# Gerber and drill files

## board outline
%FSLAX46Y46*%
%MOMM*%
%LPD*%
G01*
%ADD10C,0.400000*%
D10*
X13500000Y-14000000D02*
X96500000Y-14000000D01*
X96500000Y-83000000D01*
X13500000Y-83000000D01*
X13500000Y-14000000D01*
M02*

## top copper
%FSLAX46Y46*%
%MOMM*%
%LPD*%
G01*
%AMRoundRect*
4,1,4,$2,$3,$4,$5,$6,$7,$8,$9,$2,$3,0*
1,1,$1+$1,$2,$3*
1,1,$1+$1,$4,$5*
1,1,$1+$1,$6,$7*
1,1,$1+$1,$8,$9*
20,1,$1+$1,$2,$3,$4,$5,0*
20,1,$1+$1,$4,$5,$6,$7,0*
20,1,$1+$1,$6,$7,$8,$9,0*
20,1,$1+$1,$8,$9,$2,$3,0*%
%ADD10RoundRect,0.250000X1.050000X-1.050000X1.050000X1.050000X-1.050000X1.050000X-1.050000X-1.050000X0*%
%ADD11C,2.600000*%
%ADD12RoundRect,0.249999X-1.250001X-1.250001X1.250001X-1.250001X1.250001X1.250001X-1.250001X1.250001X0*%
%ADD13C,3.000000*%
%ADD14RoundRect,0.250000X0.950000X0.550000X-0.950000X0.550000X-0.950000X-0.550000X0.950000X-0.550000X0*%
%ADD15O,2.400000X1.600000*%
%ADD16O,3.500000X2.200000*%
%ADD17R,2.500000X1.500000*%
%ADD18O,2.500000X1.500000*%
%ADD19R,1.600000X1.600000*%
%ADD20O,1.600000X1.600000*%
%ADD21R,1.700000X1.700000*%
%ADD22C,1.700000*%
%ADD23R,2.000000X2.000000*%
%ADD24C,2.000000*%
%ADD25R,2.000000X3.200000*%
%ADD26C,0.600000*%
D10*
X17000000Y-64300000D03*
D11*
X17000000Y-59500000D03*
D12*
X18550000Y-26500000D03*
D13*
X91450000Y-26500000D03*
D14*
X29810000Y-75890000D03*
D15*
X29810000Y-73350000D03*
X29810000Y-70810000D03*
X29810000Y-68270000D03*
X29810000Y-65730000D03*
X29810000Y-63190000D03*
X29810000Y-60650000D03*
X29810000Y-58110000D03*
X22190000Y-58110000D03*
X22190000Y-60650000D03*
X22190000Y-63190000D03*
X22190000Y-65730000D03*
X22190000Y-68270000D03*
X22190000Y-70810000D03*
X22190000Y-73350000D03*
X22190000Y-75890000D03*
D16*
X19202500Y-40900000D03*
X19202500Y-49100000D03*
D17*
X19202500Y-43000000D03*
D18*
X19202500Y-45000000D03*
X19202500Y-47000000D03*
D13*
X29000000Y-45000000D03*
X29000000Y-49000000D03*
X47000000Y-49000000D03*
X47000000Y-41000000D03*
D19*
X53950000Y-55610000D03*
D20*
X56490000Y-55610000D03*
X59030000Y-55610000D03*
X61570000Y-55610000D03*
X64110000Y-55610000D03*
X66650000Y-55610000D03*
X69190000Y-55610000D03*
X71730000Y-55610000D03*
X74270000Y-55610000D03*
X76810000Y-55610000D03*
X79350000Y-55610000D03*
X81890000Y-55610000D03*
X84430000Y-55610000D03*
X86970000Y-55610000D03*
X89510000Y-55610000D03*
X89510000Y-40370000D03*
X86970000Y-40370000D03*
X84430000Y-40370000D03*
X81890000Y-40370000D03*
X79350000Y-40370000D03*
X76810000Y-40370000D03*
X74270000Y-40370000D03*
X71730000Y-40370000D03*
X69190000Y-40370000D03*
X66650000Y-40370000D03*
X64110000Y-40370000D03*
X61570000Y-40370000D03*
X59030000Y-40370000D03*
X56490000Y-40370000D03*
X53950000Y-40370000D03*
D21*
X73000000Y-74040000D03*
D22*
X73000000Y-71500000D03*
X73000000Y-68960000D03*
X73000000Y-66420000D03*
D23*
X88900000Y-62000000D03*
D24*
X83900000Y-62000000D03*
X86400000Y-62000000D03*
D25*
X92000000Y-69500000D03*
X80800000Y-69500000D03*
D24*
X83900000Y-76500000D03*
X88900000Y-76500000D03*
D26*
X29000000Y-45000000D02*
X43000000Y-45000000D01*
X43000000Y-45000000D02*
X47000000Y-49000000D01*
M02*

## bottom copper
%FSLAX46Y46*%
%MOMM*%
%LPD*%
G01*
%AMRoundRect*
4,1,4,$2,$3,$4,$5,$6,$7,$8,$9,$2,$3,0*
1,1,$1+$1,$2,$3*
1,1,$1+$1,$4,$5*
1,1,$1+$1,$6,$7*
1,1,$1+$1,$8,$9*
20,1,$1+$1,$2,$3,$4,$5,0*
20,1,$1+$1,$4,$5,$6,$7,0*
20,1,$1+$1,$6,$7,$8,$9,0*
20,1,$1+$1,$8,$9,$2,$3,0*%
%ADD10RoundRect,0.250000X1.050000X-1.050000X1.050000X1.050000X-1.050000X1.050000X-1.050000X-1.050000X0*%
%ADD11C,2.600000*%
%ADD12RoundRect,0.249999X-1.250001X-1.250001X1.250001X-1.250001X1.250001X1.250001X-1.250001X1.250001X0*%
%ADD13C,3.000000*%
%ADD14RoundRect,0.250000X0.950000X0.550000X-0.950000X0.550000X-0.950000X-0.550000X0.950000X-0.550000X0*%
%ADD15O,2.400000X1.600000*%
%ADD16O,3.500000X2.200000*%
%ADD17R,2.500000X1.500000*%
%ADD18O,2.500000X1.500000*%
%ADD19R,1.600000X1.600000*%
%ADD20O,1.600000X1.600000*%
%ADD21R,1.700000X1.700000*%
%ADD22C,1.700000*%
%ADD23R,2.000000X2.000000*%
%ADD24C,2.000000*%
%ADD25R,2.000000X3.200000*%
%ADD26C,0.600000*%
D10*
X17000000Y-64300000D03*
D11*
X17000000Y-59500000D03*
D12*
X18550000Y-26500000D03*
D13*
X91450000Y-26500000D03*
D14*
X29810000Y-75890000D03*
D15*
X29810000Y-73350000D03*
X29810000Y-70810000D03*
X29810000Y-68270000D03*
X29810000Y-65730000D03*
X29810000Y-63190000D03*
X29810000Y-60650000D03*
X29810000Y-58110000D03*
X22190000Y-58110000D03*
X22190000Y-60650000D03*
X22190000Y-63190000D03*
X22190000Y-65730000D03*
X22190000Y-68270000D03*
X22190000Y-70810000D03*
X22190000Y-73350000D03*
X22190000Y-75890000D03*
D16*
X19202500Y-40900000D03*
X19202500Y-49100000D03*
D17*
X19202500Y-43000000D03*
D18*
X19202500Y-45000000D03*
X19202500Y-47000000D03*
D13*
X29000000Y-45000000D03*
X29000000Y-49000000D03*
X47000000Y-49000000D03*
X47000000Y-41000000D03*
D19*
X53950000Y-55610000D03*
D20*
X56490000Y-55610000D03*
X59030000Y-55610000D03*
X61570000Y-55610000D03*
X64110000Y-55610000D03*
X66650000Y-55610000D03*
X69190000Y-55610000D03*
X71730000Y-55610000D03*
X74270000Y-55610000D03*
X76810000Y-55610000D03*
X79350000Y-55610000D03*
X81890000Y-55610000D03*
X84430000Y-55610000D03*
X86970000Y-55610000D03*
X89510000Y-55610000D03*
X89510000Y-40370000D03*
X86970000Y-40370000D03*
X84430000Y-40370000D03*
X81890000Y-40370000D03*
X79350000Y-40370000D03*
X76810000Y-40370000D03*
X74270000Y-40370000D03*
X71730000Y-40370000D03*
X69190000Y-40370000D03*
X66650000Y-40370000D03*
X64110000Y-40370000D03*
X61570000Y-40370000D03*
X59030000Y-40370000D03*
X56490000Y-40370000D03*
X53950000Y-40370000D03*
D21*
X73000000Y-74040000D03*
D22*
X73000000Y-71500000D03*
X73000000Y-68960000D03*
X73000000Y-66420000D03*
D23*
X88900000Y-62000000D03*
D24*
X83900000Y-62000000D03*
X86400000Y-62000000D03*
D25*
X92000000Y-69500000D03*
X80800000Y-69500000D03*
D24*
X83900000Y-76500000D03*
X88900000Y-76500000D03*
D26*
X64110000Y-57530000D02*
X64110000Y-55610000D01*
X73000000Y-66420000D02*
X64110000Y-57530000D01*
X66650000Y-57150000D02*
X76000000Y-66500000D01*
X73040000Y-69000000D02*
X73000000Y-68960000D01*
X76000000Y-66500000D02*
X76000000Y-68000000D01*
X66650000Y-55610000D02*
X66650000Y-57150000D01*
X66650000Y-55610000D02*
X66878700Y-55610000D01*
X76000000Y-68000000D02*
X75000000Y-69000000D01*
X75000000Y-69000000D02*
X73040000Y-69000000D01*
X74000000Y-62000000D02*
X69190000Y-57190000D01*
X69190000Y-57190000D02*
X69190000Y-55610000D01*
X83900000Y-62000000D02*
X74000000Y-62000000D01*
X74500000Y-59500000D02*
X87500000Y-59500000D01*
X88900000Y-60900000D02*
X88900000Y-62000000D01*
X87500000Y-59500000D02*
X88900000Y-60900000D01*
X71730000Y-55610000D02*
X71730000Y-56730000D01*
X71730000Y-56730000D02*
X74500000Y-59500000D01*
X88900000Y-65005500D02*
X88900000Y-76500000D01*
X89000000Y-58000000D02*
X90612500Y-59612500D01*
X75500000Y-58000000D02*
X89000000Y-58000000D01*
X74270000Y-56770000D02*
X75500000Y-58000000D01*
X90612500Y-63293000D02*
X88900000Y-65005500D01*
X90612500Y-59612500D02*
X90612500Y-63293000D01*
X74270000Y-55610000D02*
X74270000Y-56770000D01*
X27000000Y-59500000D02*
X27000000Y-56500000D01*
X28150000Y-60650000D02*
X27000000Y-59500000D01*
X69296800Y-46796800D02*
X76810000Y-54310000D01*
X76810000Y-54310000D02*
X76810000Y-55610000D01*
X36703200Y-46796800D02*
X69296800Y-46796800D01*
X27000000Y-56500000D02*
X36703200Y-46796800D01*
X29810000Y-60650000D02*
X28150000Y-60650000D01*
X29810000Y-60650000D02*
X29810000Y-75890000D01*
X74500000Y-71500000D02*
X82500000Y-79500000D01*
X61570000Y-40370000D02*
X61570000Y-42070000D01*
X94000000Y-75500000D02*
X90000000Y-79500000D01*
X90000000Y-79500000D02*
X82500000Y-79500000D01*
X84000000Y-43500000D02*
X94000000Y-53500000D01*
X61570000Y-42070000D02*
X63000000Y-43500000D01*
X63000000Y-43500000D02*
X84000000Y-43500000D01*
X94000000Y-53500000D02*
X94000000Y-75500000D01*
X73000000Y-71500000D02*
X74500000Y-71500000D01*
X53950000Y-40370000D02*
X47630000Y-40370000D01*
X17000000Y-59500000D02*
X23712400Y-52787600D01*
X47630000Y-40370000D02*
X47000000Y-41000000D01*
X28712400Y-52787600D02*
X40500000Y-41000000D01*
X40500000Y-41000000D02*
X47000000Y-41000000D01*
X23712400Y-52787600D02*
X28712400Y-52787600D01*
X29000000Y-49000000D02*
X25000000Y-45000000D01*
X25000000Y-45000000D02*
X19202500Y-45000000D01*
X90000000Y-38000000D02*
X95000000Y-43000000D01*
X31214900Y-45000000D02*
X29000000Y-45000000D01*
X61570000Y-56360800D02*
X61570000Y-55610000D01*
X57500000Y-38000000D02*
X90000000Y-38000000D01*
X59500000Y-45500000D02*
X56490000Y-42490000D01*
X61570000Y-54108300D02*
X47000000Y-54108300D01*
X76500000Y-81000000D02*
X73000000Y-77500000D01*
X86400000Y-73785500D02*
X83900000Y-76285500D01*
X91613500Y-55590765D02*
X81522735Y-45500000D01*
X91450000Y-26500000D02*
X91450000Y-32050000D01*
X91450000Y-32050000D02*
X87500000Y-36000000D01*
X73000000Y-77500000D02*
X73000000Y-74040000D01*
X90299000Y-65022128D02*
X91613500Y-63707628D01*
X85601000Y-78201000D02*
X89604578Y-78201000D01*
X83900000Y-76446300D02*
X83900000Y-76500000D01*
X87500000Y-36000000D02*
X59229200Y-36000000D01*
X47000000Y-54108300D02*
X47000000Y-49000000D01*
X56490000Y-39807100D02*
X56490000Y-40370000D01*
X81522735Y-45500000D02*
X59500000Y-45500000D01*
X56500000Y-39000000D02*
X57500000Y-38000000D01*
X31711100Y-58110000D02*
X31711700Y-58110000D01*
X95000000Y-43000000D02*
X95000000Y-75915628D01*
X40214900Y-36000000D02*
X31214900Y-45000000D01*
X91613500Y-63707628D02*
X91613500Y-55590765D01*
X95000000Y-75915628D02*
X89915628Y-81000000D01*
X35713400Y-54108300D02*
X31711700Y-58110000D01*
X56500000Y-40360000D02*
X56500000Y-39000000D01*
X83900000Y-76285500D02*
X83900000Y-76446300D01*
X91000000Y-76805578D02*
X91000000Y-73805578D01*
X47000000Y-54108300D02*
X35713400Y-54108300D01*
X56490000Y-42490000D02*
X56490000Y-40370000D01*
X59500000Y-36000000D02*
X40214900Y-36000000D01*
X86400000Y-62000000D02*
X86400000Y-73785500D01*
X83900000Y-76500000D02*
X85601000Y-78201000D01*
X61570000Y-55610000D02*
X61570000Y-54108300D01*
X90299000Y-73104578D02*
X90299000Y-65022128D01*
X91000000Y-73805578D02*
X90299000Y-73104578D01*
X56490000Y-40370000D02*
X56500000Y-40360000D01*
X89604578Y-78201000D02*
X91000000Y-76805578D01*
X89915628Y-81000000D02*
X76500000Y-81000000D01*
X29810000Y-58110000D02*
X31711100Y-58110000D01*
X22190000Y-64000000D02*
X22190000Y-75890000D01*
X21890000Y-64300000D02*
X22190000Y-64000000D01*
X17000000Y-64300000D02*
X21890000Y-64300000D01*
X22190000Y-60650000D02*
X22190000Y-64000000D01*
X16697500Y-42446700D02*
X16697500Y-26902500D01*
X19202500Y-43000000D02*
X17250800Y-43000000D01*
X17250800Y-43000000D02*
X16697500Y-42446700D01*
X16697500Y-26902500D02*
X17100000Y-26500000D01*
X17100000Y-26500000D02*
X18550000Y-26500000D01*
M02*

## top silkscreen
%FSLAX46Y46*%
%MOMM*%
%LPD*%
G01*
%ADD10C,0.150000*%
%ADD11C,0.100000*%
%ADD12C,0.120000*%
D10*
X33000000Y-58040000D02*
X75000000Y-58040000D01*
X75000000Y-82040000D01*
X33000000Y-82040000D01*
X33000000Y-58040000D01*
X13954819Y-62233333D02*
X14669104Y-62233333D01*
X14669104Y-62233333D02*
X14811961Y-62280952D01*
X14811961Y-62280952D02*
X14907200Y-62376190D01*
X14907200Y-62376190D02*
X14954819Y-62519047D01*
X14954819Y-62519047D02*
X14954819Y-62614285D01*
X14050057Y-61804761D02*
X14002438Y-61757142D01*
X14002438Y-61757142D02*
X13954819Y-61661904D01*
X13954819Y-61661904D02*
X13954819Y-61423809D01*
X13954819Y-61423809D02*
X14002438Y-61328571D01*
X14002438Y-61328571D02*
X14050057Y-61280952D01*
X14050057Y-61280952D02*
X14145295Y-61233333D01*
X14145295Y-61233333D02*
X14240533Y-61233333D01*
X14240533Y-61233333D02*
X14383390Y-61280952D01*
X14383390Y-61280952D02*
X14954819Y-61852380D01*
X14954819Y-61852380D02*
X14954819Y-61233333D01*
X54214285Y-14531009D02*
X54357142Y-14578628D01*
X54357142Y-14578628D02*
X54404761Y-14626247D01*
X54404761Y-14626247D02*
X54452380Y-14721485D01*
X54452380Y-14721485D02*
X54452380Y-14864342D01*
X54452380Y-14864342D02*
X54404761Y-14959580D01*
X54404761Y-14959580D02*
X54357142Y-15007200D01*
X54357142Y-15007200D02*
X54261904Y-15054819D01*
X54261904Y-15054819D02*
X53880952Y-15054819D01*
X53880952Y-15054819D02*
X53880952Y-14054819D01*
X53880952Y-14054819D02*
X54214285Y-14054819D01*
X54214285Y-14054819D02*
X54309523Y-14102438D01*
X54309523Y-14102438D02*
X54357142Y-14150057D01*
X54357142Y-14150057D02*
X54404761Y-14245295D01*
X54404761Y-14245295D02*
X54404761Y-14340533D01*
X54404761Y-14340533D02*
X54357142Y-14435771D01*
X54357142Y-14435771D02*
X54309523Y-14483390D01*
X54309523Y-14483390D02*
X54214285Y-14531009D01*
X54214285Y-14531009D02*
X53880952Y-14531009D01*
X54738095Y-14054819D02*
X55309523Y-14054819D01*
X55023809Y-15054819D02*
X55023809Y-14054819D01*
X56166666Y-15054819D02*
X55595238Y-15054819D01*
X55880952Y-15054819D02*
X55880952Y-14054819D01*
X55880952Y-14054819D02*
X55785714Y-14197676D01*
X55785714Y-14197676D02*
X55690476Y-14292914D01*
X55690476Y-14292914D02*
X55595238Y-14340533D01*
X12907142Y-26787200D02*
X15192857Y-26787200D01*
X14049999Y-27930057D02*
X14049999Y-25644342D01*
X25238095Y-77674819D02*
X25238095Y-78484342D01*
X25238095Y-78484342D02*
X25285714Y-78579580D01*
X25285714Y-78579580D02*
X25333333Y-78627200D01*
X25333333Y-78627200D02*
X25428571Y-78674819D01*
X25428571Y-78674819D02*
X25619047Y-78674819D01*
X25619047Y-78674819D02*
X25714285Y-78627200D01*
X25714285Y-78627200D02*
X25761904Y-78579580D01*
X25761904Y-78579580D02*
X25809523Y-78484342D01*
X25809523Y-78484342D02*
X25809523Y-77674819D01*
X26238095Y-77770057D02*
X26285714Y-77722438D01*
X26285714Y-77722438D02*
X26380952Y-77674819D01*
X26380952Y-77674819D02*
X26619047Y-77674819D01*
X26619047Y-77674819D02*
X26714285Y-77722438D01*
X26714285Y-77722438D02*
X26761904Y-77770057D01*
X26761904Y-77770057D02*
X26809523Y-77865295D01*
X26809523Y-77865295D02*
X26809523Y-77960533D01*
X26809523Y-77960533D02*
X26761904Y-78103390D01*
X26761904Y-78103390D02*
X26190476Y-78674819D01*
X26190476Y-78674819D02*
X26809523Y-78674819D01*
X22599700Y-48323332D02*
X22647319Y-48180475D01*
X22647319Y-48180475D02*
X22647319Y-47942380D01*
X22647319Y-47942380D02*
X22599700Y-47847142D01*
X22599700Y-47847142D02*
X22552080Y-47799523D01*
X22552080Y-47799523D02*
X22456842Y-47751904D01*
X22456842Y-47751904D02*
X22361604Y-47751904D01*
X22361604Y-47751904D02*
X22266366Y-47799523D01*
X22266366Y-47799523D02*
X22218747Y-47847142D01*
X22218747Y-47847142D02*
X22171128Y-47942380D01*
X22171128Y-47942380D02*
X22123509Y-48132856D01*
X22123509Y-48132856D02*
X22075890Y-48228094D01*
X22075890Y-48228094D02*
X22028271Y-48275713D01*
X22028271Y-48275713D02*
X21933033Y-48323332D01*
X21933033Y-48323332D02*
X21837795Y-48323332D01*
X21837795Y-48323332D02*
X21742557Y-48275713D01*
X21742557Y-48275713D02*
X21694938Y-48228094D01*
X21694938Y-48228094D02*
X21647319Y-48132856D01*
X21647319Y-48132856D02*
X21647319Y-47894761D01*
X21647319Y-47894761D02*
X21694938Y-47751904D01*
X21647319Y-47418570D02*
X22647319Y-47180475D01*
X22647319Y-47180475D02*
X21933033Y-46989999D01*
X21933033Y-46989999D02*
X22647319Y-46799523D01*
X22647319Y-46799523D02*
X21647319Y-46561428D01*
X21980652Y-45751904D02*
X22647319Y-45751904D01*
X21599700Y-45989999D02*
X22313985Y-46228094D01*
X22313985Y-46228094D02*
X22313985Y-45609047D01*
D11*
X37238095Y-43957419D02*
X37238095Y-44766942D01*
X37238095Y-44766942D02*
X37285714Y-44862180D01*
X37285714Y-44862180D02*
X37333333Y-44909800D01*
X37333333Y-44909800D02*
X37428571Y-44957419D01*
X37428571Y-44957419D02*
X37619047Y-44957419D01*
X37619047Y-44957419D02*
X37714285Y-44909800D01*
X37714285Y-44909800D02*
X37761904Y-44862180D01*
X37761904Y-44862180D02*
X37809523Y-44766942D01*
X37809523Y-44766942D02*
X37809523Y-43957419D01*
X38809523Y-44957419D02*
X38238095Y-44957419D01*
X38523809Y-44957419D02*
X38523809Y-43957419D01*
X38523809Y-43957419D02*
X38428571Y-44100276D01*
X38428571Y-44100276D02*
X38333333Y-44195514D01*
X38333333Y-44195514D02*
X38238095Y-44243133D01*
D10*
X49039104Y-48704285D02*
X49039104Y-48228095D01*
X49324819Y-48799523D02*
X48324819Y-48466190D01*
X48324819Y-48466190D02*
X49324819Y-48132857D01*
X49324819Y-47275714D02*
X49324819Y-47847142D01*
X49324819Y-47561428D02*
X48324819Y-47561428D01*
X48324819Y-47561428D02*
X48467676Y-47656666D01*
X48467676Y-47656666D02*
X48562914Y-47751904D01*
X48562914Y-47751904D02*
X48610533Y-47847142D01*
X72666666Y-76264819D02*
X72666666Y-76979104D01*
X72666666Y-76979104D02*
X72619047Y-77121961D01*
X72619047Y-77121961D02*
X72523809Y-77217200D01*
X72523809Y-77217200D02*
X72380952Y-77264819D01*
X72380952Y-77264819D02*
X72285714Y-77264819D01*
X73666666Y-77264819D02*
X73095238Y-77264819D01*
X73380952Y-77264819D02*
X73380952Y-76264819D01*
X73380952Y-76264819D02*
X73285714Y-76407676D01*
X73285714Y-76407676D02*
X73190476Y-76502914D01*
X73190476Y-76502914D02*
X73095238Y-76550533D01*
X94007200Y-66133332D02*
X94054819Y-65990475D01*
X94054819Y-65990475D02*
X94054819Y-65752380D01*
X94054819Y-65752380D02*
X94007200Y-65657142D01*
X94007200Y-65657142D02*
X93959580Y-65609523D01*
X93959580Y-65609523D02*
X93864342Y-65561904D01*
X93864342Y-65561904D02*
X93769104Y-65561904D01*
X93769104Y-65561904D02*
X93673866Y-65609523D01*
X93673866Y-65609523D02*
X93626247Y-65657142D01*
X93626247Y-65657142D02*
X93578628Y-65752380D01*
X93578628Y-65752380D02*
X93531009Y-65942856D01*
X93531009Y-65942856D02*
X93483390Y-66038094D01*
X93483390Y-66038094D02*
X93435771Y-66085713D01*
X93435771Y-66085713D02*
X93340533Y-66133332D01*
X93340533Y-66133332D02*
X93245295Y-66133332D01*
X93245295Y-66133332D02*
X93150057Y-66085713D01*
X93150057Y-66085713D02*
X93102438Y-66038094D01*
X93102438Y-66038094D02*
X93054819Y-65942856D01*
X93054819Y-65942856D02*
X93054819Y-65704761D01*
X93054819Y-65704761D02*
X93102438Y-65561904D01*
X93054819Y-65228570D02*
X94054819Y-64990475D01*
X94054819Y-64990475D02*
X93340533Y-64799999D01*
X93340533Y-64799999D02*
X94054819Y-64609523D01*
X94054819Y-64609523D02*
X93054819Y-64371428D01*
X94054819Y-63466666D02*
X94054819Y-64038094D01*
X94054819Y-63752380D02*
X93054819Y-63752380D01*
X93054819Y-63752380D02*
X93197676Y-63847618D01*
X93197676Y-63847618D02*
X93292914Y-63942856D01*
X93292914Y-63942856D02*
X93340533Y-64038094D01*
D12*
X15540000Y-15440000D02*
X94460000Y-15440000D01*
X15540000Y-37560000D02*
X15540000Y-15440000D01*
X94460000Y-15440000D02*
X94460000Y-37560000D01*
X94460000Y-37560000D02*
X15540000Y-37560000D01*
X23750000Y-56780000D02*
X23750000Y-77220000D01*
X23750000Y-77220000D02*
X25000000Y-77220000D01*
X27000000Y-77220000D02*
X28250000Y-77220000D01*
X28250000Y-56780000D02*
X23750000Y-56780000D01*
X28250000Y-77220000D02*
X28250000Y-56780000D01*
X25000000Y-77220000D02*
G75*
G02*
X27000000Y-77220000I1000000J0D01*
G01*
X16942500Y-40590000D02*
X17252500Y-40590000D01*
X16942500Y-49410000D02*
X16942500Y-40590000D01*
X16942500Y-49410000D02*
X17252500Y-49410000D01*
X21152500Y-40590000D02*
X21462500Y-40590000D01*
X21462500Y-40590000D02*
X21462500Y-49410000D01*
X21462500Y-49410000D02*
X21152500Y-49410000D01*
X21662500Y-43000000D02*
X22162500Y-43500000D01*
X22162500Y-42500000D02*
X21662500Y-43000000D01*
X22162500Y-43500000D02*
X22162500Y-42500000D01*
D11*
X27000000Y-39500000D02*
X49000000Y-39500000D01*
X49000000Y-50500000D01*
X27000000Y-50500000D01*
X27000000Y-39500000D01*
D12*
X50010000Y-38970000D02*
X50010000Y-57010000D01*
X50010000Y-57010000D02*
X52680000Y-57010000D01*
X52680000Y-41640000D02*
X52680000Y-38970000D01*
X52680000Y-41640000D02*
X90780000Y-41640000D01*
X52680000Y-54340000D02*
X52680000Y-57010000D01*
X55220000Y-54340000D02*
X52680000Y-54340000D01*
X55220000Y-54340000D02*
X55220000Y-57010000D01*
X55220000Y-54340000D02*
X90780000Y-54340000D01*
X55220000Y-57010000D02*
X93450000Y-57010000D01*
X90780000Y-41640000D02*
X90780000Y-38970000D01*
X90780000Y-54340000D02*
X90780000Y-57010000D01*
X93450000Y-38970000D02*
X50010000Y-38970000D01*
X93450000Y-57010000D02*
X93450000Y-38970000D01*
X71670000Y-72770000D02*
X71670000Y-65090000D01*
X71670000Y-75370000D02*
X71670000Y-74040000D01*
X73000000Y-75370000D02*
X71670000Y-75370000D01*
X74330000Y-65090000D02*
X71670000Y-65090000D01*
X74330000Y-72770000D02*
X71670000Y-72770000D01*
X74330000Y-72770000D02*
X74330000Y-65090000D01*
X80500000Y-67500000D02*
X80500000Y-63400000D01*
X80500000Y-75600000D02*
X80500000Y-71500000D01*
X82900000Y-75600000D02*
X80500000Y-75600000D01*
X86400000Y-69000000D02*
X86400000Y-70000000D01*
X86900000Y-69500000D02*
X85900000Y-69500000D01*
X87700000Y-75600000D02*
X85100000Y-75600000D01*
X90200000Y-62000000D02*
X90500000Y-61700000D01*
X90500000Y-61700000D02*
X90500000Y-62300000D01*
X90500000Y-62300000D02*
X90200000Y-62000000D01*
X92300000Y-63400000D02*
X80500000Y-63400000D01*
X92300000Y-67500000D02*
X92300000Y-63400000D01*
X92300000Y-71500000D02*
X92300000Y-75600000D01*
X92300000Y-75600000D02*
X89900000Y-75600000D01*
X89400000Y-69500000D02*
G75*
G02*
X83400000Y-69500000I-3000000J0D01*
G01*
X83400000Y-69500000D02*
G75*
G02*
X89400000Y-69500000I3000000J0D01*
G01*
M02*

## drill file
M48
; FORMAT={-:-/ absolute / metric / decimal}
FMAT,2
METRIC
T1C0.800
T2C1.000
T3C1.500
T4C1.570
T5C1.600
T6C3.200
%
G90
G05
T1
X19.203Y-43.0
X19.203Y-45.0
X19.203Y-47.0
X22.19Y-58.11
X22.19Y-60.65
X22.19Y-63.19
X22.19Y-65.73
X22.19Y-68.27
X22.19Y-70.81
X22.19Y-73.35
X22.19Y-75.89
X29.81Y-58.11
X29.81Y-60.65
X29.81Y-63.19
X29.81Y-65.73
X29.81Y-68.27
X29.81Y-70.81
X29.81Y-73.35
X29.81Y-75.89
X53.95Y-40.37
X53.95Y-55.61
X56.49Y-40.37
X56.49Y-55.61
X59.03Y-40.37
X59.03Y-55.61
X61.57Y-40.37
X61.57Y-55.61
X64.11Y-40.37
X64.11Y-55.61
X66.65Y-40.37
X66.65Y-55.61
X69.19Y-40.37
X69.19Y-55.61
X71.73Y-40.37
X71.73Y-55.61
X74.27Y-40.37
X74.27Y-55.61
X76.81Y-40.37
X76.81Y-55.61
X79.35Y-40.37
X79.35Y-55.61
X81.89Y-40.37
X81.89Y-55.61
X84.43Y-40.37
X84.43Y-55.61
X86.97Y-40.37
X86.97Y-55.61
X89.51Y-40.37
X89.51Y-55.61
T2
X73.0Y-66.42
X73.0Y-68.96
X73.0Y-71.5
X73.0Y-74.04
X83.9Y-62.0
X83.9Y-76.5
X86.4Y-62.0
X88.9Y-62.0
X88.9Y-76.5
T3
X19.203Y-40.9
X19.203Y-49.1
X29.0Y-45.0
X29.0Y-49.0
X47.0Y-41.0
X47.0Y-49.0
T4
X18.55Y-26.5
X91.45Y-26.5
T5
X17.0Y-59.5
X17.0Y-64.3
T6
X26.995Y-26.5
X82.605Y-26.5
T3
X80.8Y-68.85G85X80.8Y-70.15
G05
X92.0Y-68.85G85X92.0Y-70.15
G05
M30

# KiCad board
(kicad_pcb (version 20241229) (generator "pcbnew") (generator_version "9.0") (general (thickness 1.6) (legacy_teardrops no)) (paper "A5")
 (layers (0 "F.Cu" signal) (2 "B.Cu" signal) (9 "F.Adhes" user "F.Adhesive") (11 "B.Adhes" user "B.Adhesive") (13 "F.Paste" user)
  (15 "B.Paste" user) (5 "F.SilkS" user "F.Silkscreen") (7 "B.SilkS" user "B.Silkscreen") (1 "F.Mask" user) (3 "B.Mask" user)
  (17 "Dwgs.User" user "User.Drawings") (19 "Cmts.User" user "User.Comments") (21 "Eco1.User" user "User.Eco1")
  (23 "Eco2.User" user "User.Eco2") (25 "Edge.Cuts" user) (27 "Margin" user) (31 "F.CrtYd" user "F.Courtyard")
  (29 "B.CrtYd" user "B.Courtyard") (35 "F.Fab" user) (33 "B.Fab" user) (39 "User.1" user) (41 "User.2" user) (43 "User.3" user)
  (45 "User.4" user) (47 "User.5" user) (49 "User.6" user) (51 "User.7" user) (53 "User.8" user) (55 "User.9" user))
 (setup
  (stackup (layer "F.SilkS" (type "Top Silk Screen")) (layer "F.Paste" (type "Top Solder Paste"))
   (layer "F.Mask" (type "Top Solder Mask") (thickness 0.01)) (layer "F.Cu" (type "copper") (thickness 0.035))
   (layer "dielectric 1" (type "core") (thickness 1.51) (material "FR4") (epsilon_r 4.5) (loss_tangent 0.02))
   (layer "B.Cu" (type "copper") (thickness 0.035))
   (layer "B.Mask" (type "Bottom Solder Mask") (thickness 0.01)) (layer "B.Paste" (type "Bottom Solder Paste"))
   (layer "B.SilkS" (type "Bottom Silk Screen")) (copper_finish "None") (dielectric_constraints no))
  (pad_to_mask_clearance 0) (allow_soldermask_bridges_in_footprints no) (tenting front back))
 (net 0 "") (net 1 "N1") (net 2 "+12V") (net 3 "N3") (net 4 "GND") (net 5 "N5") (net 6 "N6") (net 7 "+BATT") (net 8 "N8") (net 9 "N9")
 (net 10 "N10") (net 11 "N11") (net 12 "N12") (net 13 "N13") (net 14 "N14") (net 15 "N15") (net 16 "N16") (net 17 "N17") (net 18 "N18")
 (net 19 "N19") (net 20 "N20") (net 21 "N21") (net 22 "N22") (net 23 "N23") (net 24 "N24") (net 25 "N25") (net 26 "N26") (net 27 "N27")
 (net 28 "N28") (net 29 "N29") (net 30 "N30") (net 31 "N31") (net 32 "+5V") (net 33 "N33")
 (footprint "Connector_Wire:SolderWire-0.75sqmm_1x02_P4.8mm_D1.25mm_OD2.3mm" (layer "F.Cu") (at 17 64.3 90)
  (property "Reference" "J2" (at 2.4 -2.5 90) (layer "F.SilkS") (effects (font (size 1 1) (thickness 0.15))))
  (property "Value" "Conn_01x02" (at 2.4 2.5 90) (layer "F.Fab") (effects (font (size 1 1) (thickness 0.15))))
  (pad "1" thru_hole roundrect (at 0 0 90) (size 2.6 2.6) (drill 1.6) (layers "*.Cu" "*.Mask") (remove_unused_layers no)
   (roundrect_rratio 0.096154) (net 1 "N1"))
  (pad "2" thru_hole circle (at 4.8 0 90) (size 2.6 2.6) (drill 1.6) (layers "*.Cu" "*.Mask") (remove_unused_layers no) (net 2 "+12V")))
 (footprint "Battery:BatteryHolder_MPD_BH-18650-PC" (layer "F.Cu") (at 18.55 26.5)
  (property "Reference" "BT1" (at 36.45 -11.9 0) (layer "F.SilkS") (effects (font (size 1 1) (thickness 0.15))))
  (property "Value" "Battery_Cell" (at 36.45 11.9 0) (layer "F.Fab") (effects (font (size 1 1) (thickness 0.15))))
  (fp_line (start -3.01 -11.06) (end 75.91 -11.06) (stroke (width 0.12) (type solid)) (layer "F.SilkS"))
  (fp_line (start -3.01 11.06) (end -3.01 -11.06) (stroke (width 0.12) (type solid)) (layer "F.SilkS"))
  (fp_line (start 75.91 -11.06) (end 75.91 11.06) (stroke (width 0.12) (type solid)) (layer "F.SilkS"))
  (fp_line (start 75.91 11.06) (end -3.01 11.06) (stroke (width 0.12) (type solid)) (layer "F.SilkS"))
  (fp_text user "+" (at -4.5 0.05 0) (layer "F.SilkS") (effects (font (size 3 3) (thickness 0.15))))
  (pad "" np_thru_hole circle (at 8.445 0) (size 3.2 3.2) (drill 3.2) (layers "*.Cu" "*.Mask"))
  (pad "" np_thru_hole circle (at 64.055 0) (size 3.2 3.2) (drill 3.2) (layers "*.Cu" "*.Mask"))
  (pad "1" thru_hole roundrect (at 0 0) (size 3 3) (drill 1.57) (layers "*.Cu" "*.Mask") (remove_unused_layers no)
   (roundrect_rratio 0.083333) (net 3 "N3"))
  (pad "2" thru_hole circle (at 72.9 0) (size 3 3) (drill 1.57) (layers "*.Cu" "*.Mask") (remove_unused_layers no) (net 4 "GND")))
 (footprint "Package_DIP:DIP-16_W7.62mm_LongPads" (layer "F.Cu") (at 29.81 75.89 180)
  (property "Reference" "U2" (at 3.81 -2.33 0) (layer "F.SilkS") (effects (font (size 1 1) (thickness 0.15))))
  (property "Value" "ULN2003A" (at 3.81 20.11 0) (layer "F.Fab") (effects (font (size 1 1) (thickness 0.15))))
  (fp_line (start 6.06 19.11) (end 6.06 -1.33) (stroke (width 0.12) (type solid)) (layer "F.SilkS"))
  (fp_line (start 6.06 -1.33) (end 4.81 -1.33) (stroke (width 0.12) (type solid)) (layer "F.SilkS"))
  (fp_line (start 2.81 -1.33) (end 1.56 -1.33) (stroke (width 0.12) (type solid)) (layer "F.SilkS"))
  (fp_line (start 1.56 19.11) (end 6.06 19.11) (stroke (width 0.12) (type solid)) (layer "F.SilkS"))
  (fp_line (start 1.56 -1.33) (end 1.56 19.11) (stroke (width 0.12) (type solid)) (layer "F.SilkS"))
  (fp_arc (start 4.81 -1.33) (mid 3.81 -0.33) (end 2.81 -1.33) (stroke (width 0.12) (type solid)) (layer "F.SilkS"))
  (pad "1" thru_hole roundrect (at 0 0 180) (size 2.4 1.6) (drill 0.8) (layers "*.Cu" "*.Mask") (remove_unused_layers no)
   (roundrect_rratio 0.15625) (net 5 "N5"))
  (pad "2" thru_hole oval (at 0 2.54 180) (size 2.4 1.6) (drill 0.8) (layers "*.Cu" "*.Mask") (remove_unused_layers no) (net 5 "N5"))
  (pad "3" thru_hole oval (at 0 5.08 180) (size 2.4 1.6) (drill 0.8) (layers "*.Cu" "*.Mask") (remove_unused_layers no) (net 5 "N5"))
  (pad "4" thru_hole oval (at 0 7.62 180) (size 2.4 1.6) (drill 0.8) (layers "*.Cu" "*.Mask") (remove_unused_layers no) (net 5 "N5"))
  (pad "5" thru_hole oval (at 0 10.16 180) (size 2.4 1.6) (drill 0.8) (layers "*.Cu" "*.Mask") (remove_unused_layers no) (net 5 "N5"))
  (pad "6" thru_hole oval (at 0 12.7 180) (size 2.4 1.6) (drill 0.8) (layers "*.Cu" "*.Mask") (remove_unused_layers no) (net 5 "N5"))
  (pad "7" thru_hole oval (at 0 15.24 180) (size 2.4 1.6) (drill 0.8) (layers "*.Cu" "*.Mask") (remove_unused_layers no) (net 5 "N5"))
  (pad "8" thru_hole oval (at 0 17.78 180) (size 2.4 1.6) (drill 0.8) (layers "*.Cu" "*.Mask") (remove_unused_layers no) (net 4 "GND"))
  (pad "9" thru_hole oval (at 7.62 17.78 180) (size 2.4 1.6) (drill 0.8) (layers "*.Cu" "*.Mask") (remove_unused_layers no) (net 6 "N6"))
  (pad "10" thru_hole oval (at 7.62 15.24 180) (size 2.4 1.6) (drill 0.8) (layers "*.Cu" "*.Mask") (remove_unused_layers no) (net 1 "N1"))
  (pad "11" thru_hole oval (at 7.62 12.7 180) (size 2.4 1.6) (drill 0.8) (layers "*.Cu" "*.Mask") (remove_unused_layers no) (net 1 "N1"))
  (pad "12" thru_hole oval (at 7.62 10.16 180) (size 2.4 1.6) (drill 0.8) (layers "*.Cu" "*.Mask") (remove_unused_layers no) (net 1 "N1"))
  (pad "13" thru_hole oval (at 7.62 7.62 180) (size 2.4 1.6) (drill 0.8) (layers "*.Cu" "*.Mask") (remove_unused_layers no) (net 1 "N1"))
  (pad "14" thru_hole oval (at 7.62 5.08 180) (size 2.4 1.6) (drill 0.8) (layers "*.Cu" "*.Mask") (remove_unused_layers no) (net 1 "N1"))
  (pad "15" thru_hole oval (at 7.62 2.54 180) (size 2.4 1.6) (drill 0.8) (layers "*.Cu" "*.Mask") (remove_unused_layers no) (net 1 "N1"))
  (pad "16" thru_hole oval (at 7.62 0 180) (size 2.4 1.6) (drill 0.8) (layers "*.Cu" "*.Mask") (remove_unused_layers no) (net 1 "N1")))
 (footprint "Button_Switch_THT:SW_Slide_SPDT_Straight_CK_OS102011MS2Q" (layer "F.Cu") (at 19.2025 43 -90)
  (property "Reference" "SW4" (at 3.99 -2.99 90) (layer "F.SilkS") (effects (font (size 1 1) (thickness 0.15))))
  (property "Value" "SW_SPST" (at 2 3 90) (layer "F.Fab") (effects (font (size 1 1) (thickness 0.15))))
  (fp_line (start -2.41 2.26) (end -2.41 1.95) (stroke (width 0.12) (type solid)) (layer "F.SilkS"))
  (fp_line (start 6.41 2.26) (end -2.41 2.26) (stroke (width 0.12) (type solid)) (layer "F.SilkS"))
  (fp_line (start 6.41 2.26) (end 6.41 1.95) (stroke (width 0.12) (type solid)) (layer "F.SilkS"))
  (fp_line (start -2.41 -1.95) (end -2.41 -2.26) (stroke (width 0.12) (type solid)) (layer "F.SilkS"))
  (fp_line (start -2.41 -2.26) (end 6.41 -2.26) (stroke (width 0.12) (type solid)) (layer "F.SilkS"))
  (fp_line (start 6.41 -2.26) (end 6.41 -1.95) (stroke (width 0.12) (type solid)) (layer "F.SilkS"))
  (fp_line (start 0 -2.46) (end 0.5 -2.96) (stroke (width 0.12) (type solid)) (layer "F.SilkS"))
  (fp_line (start -0.5 -2.96) (end 0 -2.46) (stroke (width 0.12) (type solid)) (layer "F.SilkS"))
  (fp_line (start 0.5 -2.96) (end -0.5 -2.96) (stroke (width 0.12) (type solid)) (layer "F.SilkS"))
  (pad "" thru_hole oval (at -2.1 0 270) (size 2.2 3.5) (drill 1.5) (layers "*.Cu" "*.Mask") (remove_unused_layers no))
  (pad "" thru_hole oval (at 6.1 0 270) (size 2.2 3.5) (drill 1.5) (layers "*.Cu" "*.Mask") (remove_unused_layers no))
  (pad "1" thru_hole rect (at 0 0 270) (size 1.5 2.5) (drill 0.8) (layers "*.Cu" "*.Mask") (remove_unused_layers no) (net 3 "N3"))
  (pad "2" thru_hole oval (at 2 0 270) (size 1.5 2.5) (drill 0.8) (layers "*.Cu" "*.Mask") (remove_unused_layers no) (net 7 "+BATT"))
  (pad "3" thru_hole oval (at 4 0 270) (size 1.5 2.5) (drill 0.8) (layers "*.Cu" "*.Mask") (remove_unused_layers no)))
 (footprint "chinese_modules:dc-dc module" (layer "F.Cu") (at 38 45)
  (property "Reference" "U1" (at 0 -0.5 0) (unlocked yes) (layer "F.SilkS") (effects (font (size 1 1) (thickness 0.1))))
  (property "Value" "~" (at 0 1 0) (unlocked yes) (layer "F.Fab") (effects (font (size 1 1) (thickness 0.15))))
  (fp_rect (start -11 -5.5) (end 11 5.5) (stroke (width 0.1) (type solid)) (fill no) (layer "F.SilkS"))
  (pad "1" thru_hole circle (at -9 0) (size 3 3) (drill 1.5) (layers "*.Cu" "*.Mask") (remove_unused_layers no) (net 4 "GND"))
  (pad "2" thru_hole circle (at -9 4) (size 3 3) (drill 1.5) (layers "*.Cu" "*.Mask") (remove_unused_layers no) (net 7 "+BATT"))
  (pad "3" thru_hole circle (at 9 4) (size 3 3) (drill 1.5) (layers "*.Cu" "*.Mask") (remove_unused_layers no) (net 4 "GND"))
  (pad "4" thru_hole circle (at 9 -4) (size 3 3) (drill 1.5) (layers "*.Cu" "*.Mask") (remove_unused_layers no) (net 2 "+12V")))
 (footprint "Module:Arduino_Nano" (layer "F.Cu") (at 53.95 55.61 90)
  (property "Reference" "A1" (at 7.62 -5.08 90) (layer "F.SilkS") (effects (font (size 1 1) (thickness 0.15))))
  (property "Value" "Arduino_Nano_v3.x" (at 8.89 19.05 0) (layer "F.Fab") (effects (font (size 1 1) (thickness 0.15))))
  (fp_line (start 16.64 -3.94) (end -1.4 -3.94) (stroke (width 0.12) (type solid)) (layer "F.SilkS"))
  (fp_line (start -1.4 -3.94) (end -1.4 -1.27) (stroke (width 0.12) (type solid)) (layer "F.SilkS"))
  (fp_line (start 13.97 -1.27) (end 16.64 -1.27) (stroke (width 0.12) (type solid)) (layer "F.SilkS"))
  (fp_line (start 13.97 -1.27) (end 13.97 36.83) (stroke (width 0.12) (type solid)) (layer "F.SilkS"))
  (fp_line (start 1.27 -1.27) (end -1.4 -1.27) (stroke (width 0.12) (type solid)) (layer "F.SilkS"))
  (fp_line (start 1.27 1.27) (end 1.27 -1.27) (stroke (width 0.12) (type solid)) (layer "F.SilkS"))
  (fp_line (start 1.27 1.27) (end -1.4 1.27) (stroke (width 0.12) (type solid)) (layer "F.SilkS"))
  (fp_line (start 1.27 1.27) (end 1.27 36.83) (stroke (width 0.12) (type solid)) (layer "F.SilkS"))
  (fp_line (start -1.4 1.27) (end -1.4 39.5) (stroke (width 0.12) (type solid)) (layer "F.SilkS"))
  (fp_line (start 13.97 36.83) (end 16.64 36.83) (stroke (width 0.12) (type solid)) (layer "F.SilkS"))
  (fp_line (start 1.27 36.83) (end -1.4 36.83) (stroke (width 0.12) (type solid)) (layer "F.SilkS"))
  (fp_line (start 16.64 39.5) (end 16.64 -3.94) (stroke (width 0.12) (type solid)) (layer "F.SilkS"))
  (fp_line (start -1.4 39.5) (end 16.64 39.5) (stroke (width 0.12) (type solid)) (layer "F.SilkS"))
  (pad "1" thru_hole rect (at 0 0 90) (size 1.6 1.6) (drill 0.8) (layers "*.Cu" "*.Mask") (remove_unused_layers no) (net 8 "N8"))
  (pad "2" thru_hole oval (at 0 2.54 90) (size 1.6 1.6) (drill 0.8) (layers "*.Cu" "*.Mask") (remove_unused_layers no) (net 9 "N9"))
  (pad "3" thru_hole oval (at 0 5.08 90) (size 1.6 1.6) (drill 0.8) (layers "*.Cu" "*.Mask") (remove_unused_layers no) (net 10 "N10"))
  (pad "4" thru_hole oval (at 0 7.62 90) (size 1.6 1.6) (drill 0.8) (layers "*.Cu" "*.Mask") (remove_unused_layers no) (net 4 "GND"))
  (pad "5" thru_hole oval (at 0 10.16 90) (size 1.6 1.6) (drill 0.8) (layers "*.Cu" "*.Mask") (remove_unused_layers no) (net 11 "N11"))
  (pad "6" thru_hole oval (at 0 12.7 90) (size 1.6 1.6) (drill 0.8) (layers "*.Cu" "*.Mask") (remove_unused_layers no) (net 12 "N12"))
  (pad "7" thru_hole oval (at 0 15.24 90) (size 1.6 1.6) (drill 0.8) (layers "*.Cu" "*.Mask") (remove_unused_layers no) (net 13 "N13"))
  (pad "8" thru_hole oval (at 0 17.78 90) (size 1.6 1.6) (drill 0.8) (layers "*.Cu" "*.Mask") (remove_unused_layers no) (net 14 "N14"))
  (pad "9" thru_hole oval (at 0 20.32 90) (size 1.6 1.6) (drill 0.8) (layers "*.Cu" "*.Mask") (remove_unused_layers no) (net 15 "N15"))
  (pad "10" thru_hole oval (at 0 22.86 90) (size 1.6 1.6) (drill 0.8) (layers "*.Cu" "*.Mask") (remove_unused_layers no) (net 5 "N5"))
  (pad "11" thru_hole oval (at 0 25.4 90) (size 1.6 1.6) (drill 0.8) (layers "*.Cu" "*.Mask") (remove_unused_layers no) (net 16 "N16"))
  (pad "12" thru_hole oval (at 0 27.94 90) (size 1.6 1.6) (drill 0.8) (layers "*.Cu" "*.Mask") (remove_unused_layers no) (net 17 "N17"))
  (pad "13" thru_hole oval (at 0 30.48 90) (size 1.6 1.6) (drill 0.8) (layers "*.Cu" "*.Mask") (remove_unused_layers no) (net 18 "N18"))
  (pad "14" thru_hole oval (at 0 33.02 90) (size 1.6 1.6) (drill 0.8) (layers "*.Cu" "*.Mask") (remove_unused_layers no) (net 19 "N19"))
  (pad "15" thru_hole oval (at 0 35.56 90) (size 1.6 1.6) (drill 0.8) (layers "*.Cu" "*.Mask") (remove_unused_layers no) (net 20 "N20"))
  (pad "16" thru_hole oval (at 15.24 35.56 90) (size 1.6 1.6) (drill 0.8) (layers "*.Cu" "*.Mask") (remove_unused_layers no) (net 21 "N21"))
  (pad "17" thru_hole oval (at 15.24 33.02 90) (size 1.6 1.6) (drill 0.8) (layers "*.Cu" "*.Mask") (remove_unused_layers no) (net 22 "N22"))
  (pad "18" thru_hole oval (at 15.24 30.48 90) (size 1.6 1.6) (drill 0.8) (layers "*.Cu" "*.Mask") (remove_unused_layers no) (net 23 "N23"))
  (pad "19" thru_hole oval (at 15.24 27.94 90) (size 1.6 1.6) (drill 0.8) (layers "*.Cu" "*.Mask") (remove_unused_layers no) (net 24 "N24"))
  (pad "20" thru_hole oval (at 15.24 25.4 90) (size 1.6 1.6) (drill 0.8) (layers "*.Cu" "*.Mask") (remove_unused_layers no) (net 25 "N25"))
  (pad "21" thru_hole oval (at 15.24 22.86 90) (size 1.6 1.6) (drill 0.8) (layers "*.Cu" "*.Mask") (remove_unused_layers no) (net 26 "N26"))
  (pad "22" thru_hole oval (at 15.24 20.32 90) (size 1.6 1.6) (drill 0.8) (layers "*.Cu" "*.Mask") (remove_unused_layers no) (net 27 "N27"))
  (pad "23" thru_hole oval (at 15.24 17.78 90) (size 1.6 1.6) (drill 0.8) (layers "*.Cu" "*.Mask") (remove_unused_layers no) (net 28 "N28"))
  (pad "24" thru_hole oval (at 15.24 15.24 90) (size 1.6 1.6) (drill 0.8) (layers "*.Cu" "*.Mask") (remove_unused_layers no) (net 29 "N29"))
  (pad "25" thru_hole oval (at 15.24 12.7 90) (size 1.6 1.6) (drill 0.8) (layers "*.Cu" "*.Mask") (remove_unused_layers no) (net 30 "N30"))
  (pad "26" thru_hole oval (at 15.24 10.16 90) (size 1.6 1.6) (drill 0.8) (layers "*.Cu" "*.Mask") (remove_unused_layers no) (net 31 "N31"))
  (pad "27" thru_hole oval (at 15.24 7.62 90) (size 1.6 1.6) (drill 0.8) (layers "*.Cu" "*.Mask") (remove_unused_layers no) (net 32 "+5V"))
  (pad "28" thru_hole oval (at 15.24 5.08 90) (size 1.6 1.6) (drill 0.8) (layers "*.Cu" "*.Mask") (remove_unused_layers no) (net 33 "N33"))
  (pad "29" thru_hole oval (at 15.24 2.54 90) (size 1.6 1.6) (drill 0.8) (layers "*.Cu" "*.Mask") (remove_unused_layers no) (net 4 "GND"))
  (pad "30" thru_hole oval (at 15.24 0 90) (size 1.6 1.6) (drill 0.8) (layers "*.Cu" "*.Mask") (remove_unused_layers no) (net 2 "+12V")))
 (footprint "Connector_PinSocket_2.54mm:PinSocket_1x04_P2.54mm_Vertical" (layer "F.Cu") (at 73 74.04 180)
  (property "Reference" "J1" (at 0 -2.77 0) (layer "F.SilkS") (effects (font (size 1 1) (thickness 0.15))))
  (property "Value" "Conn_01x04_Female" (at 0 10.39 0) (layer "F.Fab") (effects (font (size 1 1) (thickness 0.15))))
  (fp_line (start 1.33 1.27) (end 1.33 8.95) (stroke (width 0.12) (type solid)) (layer "F.SilkS"))
  (fp_line (start 1.33 -1.33) (end 1.33 0) (stroke (width 0.12) (type solid)) (layer "F.SilkS"))
  (fp_line (start 0 -1.33) (end 1.33 -1.33) (stroke (width 0.12) (type solid)) (layer "F.SilkS"))
  (fp_line (start -1.33 8.95) (end 1.33 8.95) (stroke (width 0.12) (type solid)) (layer "F.SilkS"))
  (fp_line (start -1.33 1.27) (end 1.33 1.27) (stroke (width 0.12) (type solid)) (layer "F.SilkS"))
  (fp_line (start -1.33 1.27) (end -1.33 8.95) (stroke (width 0.12) (type solid)) (layer "F.SilkS"))
  (pad "1" thru_hole rect (at 0 0 180) (size 1.7 1.7) (drill 1) (layers "*.Cu" "*.Mask") (remove_unused_layers no) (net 4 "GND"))
  (pad "2" thru_hole circle (at 0 2.54 180) (size 1.7 1.7) (drill 1) (layers "*.Cu" "*.Mask") (remove_unused_layers no) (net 32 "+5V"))
  (pad "3" thru_hole circle (at 0 5.08 180) (size 1.7 1.7) (drill 1) (layers "*.Cu" "*.Mask") (remove_unused_layers no) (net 12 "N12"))
  (pad "4" thru_hole circle (at 0 7.62 180) (size 1.7 1.7) (drill 1) (layers "*.Cu" "*.Mask") (remove_unused_layers no) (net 11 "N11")))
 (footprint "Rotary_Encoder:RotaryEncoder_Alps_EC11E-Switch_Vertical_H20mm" (layer "F.Cu") (at 88.9 62 -90)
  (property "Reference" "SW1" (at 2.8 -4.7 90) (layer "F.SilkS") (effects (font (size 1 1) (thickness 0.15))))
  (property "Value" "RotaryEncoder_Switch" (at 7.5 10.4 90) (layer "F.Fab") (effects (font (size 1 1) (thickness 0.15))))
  (fp_line (start 5.5 8.4) (end 1.4 8.4) (stroke (width 0.12) (type solid)) (layer "F.SilkS"))
  (fp_line (start 13.6 8.4) (end 9.5 8.4) (stroke (width 0.12) (type solid)) (layer "F.SilkS"))
  (fp_line (start 13.6 6) (end 13.6 8.4) (stroke (width 0.12) (type solid)) (layer "F.SilkS"))
  (fp_line (start 7 2.5) (end 8 2.5) (stroke (width 0.12) (type solid)) (layer "F.SilkS"))
  (fp_line (start 7.5 2) (end 7.5 3) (stroke (width 0.12) (type solid)) (layer "F.SilkS"))
  (fp_line (start 13.6 1.2) (end 13.6 3.8) (stroke (width 0.12) (type solid)) (layer "F.SilkS"))
  (fp_line (start 0 -1.3) (end -0.3 -1.6) (stroke (width 0.12) (type solid)) (layer "F.SilkS"))
  (fp_line (start -0.3 -1.6) (end 0.3 -1.6) (stroke (width 0.12) (type solid)) (layer "F.SilkS"))
  (fp_line (start 0.3 -1.6) (end 0 -1.3) (stroke (width 0.12) (type solid)) (layer "F.SilkS"))
  (fp_line (start 1.4 -3.4) (end 1.4 8.4) (stroke (width 0.12) (type solid)) (layer "F.SilkS"))
  (fp_line (start 5.5 -3.4) (end 1.4 -3.4) (stroke (width 0.12) (type solid)) (layer "F.SilkS"))
  (fp_line (start 9.5 -3.4) (end 13.6 -3.4) (stroke (width 0.12) (type solid)) (layer "F.SilkS"))
  (fp_line (start 13.6 -3.4) (end 13.6 -1) (stroke (width 0.12) (type solid)) (layer "F.SilkS"))
  (fp_circle (center 7.5 2.5) (end 10.5 2.5) (stroke (width 0.12) (type solid)) (fill no) (layer "F.SilkS"))
  (pad "A" thru_hole rect (at 0 0 270) (size 2 2) (drill 1) (layers "*.Cu" "*.Mask") (remove_unused_layers no) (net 14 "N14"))
  (pad "B" thru_hole circle (at 0 5 270) (size 2 2) (drill 1) (layers "*.Cu" "*.Mask") (remove_unused_layers no) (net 13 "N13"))
  (pad "C" thru_hole circle (at 0 2.5 270) (size 2 2) (drill 1) (layers "*.Cu" "*.Mask") (remove_unused_layers no) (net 4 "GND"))
  (pad "MP" thru_hole rect (at 7.5 -3.1 270) (size 3.2 2) (drill oval 2.8 1.5) (layers "*.Cu" "*.Mask") (remove_unused_layers no))
  (pad "MP" thru_hole rect (at 7.5 8.1 270) (size 3.2 2) (drill oval 2.8 1.5) (layers "*.Cu" "*.Mask") (remove_unused_layers no))
  (pad "S1" thru_hole circle (at 14.5 5 270) (size 2 2) (drill 1) (layers "*.Cu" "*.Mask") (remove_unused_layers no) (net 4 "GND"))
  (pad "S2" thru_hole circle (at 14.5 0 270) (size 2 2) (drill 1) (layers "*.Cu" "*.Mask") (remove_unused_layers no) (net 15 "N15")))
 (gr_rect (start 33 58.04) (end 75 82.04) (stroke (width 0.15) (type default)) (fill no) (layer "F.SilkS"))
 (gr_rect (start 13.5 14) (end 96.5 83) (stroke (width 0.4) (type solid)) (fill no) (layer "Edge.Cuts"))
 (segment (start 64.11 57.53) (end 64.11 55.61) (width 0.6) (layer "B.Cu") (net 11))
 (segment (start 73 66.42) (end 64.11 57.53) (width 0.6) (layer "B.Cu") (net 11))
 (segment (start 66.65 57.15) (end 76 66.5) (width 0.6) (layer "B.Cu") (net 12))
 (segment (start 73.04 69) (end 73 68.96) (width 0.6) (layer "B.Cu") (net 12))
 (segment (start 76 66.5) (end 76 68) (width 0.6) (layer "B.Cu") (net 12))
 (segment (start 66.65 55.61) (end 66.65 57.15) (width 0.6) (layer "B.Cu") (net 12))
 (segment (start 66.65 55.61) (end 66.8787 55.61) (width 0.6) (layer "B.Cu") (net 12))
 (segment (start 76 68) (end 75 69) (width 0.6) (layer "B.Cu") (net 12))
 (segment (start 75 69) (end 73.04 69) (width 0.6) (layer "B.Cu") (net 12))
 (segment (start 74 62) (end 69.19 57.19) (width 0.6) (layer "B.Cu") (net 13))
 (segment (start 69.19 57.19) (end 69.19 55.61) (width 0.6) (layer "B.Cu") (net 13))
 (segment (start 83.9 62) (end 74 62) (width 0.6) (layer "B.Cu") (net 13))
 (segment (start 74.5 59.5) (end 87.5 59.5) (width 0.6) (layer "B.Cu") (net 14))
 (segment (start 88.9 60.9) (end 88.9 62) (width 0.6) (layer "B.Cu") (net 14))
 (segment (start 87.5 59.5) (end 88.9 60.9) (width 0.6) (layer "B.Cu") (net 14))
 (segment (start 71.73 55.61) (end 71.73 56.73) (width 0.6) (layer "B.Cu") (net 14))
 (segment (start 71.73 56.73) (end 74.5 59.5) (width 0.6) (layer "B.Cu") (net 14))
 (segment (start 88.9 65.0055) (end 88.9 76.5) (width 0.6) (layer "B.Cu") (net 15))
 (segment (start 89 58) (end 90.6125 59.6125) (width 0.6) (layer "B.Cu") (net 15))
 (segment (start 75.5 58) (end 89 58) (width 0.6) (layer "B.Cu") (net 15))
 (segment (start 74.27 56.77) (end 75.5 58) (width 0.6) (layer "B.Cu") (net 15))
 (segment (start 90.6125 63.293) (end 88.9 65.0055) (width 0.6) (layer "B.Cu") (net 15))
 (segment (start 90.6125 59.6125) (end 90.6125 63.293) (width 0.6) (layer "B.Cu") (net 15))
 (segment (start 74.27 55.61) (end 74.27 56.77) (width 0.6) (layer "B.Cu") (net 15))
 (segment (start 27 59.5) (end 27 56.5) (width 0.6) (layer "B.Cu") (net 5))
 (segment (start 28.15 60.65) (end 27 59.5) (width 0.6) (layer "B.Cu") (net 5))
 (segment (start 69.2968 46.7968) (end 76.81 54.31) (width 0.6) (layer "B.Cu") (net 5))
 (segment (start 76.81 54.31) (end 76.81 55.61) (width 0.6) (layer "B.Cu") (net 5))
 (segment (start 36.7032 46.7968) (end 69.2968 46.7968) (width 0.6) (layer "B.Cu") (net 5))
 (segment (start 27 56.5) (end 36.7032 46.7968) (width 0.6) (layer "B.Cu") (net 5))
 (segment (start 29.81 60.65) (end 28.15 60.65) (width 0.6) (layer "B.Cu") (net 5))
 (segment (start 29.81 60.65) (end 29.81 75.89) (width 0.6) (layer "B.Cu") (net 5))
 (segment (start 74.5 71.5) (end 82.5 79.5) (width 0.6) (layer "B.Cu") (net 32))
 (segment (start 61.57 40.37) (end 61.57 42.07) (width 0.6) (layer "B.Cu") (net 32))
 (segment (start 94 75.5) (end 90 79.5) (width 0.6) (layer "B.Cu") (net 32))
 (segment (start 90 79.5) (end 82.5 79.5) (width 0.6) (layer "B.Cu") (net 32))
 (segment (start 84 43.5) (end 94 53.5) (width 0.6) (layer "B.Cu") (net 32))
 (segment (start 61.57 42.07) (end 63 43.5) (width 0.6) (layer "B.Cu") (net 32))
 (segment (start 63 43.5) (end 84 43.5) (width 0.6) (layer "B.Cu") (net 32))
 (segment (start 94 53.5) (end 94 75.5) (width 0.6) (layer "B.Cu") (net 32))
 (segment (start 73 71.5) (end 74.5 71.5) (width 0.6) (layer "B.Cu") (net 32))
 (segment (start 53.95 40.37) (end 47.63 40.37) (width 0.6) (layer "B.Cu") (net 2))
 (segment (start 17 59.5) (end 23.7124 52.7876) (width 0.6) (layer "B.Cu") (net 2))
 (segment (start 47.63 40.37) (end 47 41) (width 0.6) (layer "B.Cu") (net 2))
 (segment (start 28.7124 52.7876) (end 40.5 41) (width 0.6) (layer "B.Cu") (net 2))
 (segment (start 40.5 41) (end 47 41) (width 0.6) (layer "B.Cu") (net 2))
 (segment (start 23.7124 52.7876) (end 28.7124 52.7876) (width 0.6) (layer "B.Cu") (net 2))
 (segment (start 29 49) (end 25 45) (width 0.6) (layer "B.Cu") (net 7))
 (segment (start 25 45) (end 19.2025 45) (width 0.6) (layer "B.Cu") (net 7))
 (segment (start 29 45) (end 43 45) (width 0.6) (layer "F.Cu") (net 4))
 (segment (start 43 45) (end 47 49) (width 0.6) (layer "F.Cu") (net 4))
 (segment (start 90 38) (end 95 43) (width 0.6) (layer "B.Cu") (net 4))
 (segment (start 31.2149 45) (end 29 45) (width 0.6) (layer "B.Cu") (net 4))
 (segment (start 61.57 56.3608) (end 61.57 55.61) (width 0.6) (layer "B.Cu") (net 4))
 (segment (start 57.5 38) (end 90 38) (width 0.6) (layer "B.Cu") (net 4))
 (segment (start 59.5 45.5) (end 56.49 42.49) (width 0.6) (layer "B.Cu") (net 4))
 (segment (start 61.57 54.1083) (end 47 54.1083) (width 0.6) (layer "B.Cu") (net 4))
 (segment (start 76.5 81) (end 73 77.5) (width 0.6) (layer "B.Cu") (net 4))
 (segment (start 86.4 73.7855) (end 83.9 76.2855) (width 0.6) (layer "B.Cu") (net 4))
 (segment (start 91.6135 55.590765) (end 81.522735 45.5) (width 0.6) (layer "B.Cu") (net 4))
 (segment (start 91.45 26.5) (end 91.45 32.05) (width 0.6) (layer "B.Cu") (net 4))
 (segment (start 91.45 32.05) (end 87.5 36) (width 0.6) (layer "B.Cu") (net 4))
 (segment (start 73 77.5) (end 73 74.04) (width 0.6) (layer "B.Cu") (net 4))
 (segment (start 90.299 65.022128) (end 91.6135 63.707628) (width 0.6) (layer "B.Cu") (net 4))
 (segment (start 85.601 78.201) (end 89.604578 78.201) (width 0.6) (layer "B.Cu") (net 4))
 (segment (start 83.9 76.4463) (end 83.9 76.5) (width 0.6) (layer "B.Cu") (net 4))
 (segment (start 87.5 36) (end 59.2292 36) (width 0.6) (layer "B.Cu") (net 4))
 (segment (start 47 54.1083) (end 47 49) (width 0.6) (layer "B.Cu") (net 4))
 (segment (start 56.49 39.8071) (end 56.49 40.37) (width 0.6) (layer "B.Cu") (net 4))
 (segment (start 81.522735 45.5) (end 59.5 45.5) (width 0.6) (layer "B.Cu") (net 4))
 (segment (start 56.5 39) (end 57.5 38) (width 0.6) (layer "B.Cu") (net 4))
 (segment (start 31.7111 58.11) (end 31.7117 58.11) (width 0.6) (layer "B.Cu") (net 4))
 (segment (start 95 43) (end 95 75.915628) (width 0.6) (layer "B.Cu") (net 4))
 (segment (start 40.2149 36) (end 31.2149 45) (width 0.6) (layer "B.Cu") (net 4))
 (segment (start 91.6135 63.707628) (end 91.6135 55.590765) (width 0.6) (layer "B.Cu") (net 4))
 (segment (start 95 75.915628) (end 89.915628 81) (width 0.6) (layer "B.Cu") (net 4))
 (segment (start 35.7134 54.1083) (end 31.7117 58.11) (width 0.6) (layer "B.Cu") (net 4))
 (segment (start 56.5 40.36) (end 56.5 39) (width 0.6) (layer "B.Cu") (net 4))
 (segment (start 83.9 76.2855) (end 83.9 76.4463) (width 0.6) (layer "B.Cu") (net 4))
 (segment (start 91 76.805578) (end 91 73.805578) (width 0.6) (layer "B.Cu") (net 4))
 (segment (start 47 54.1083) (end 35.7134 54.1083) (width 0.6) (layer "B.Cu") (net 4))
 (segment (start 56.49 42.49) (end 56.49 40.37) (width 0.6) (layer "B.Cu") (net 4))
 (segment (start 59.5 36) (end 40.2149 36) (width 0.6) (layer "B.Cu") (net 4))
 (segment (start 86.4 62) (end 86.4 73.7855) (width 0.6) (layer "B.Cu") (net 4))
 (segment (start 83.9 76.5) (end 85.601 78.201) (width 0.6) (layer "B.Cu") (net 4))
 (segment (start 61.57 55.61) (end 61.57 54.1083) (width 0.6) (layer "B.Cu") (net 4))
 (segment (start 90.299 73.104578) (end 90.299 65.022128) (width 0.6) (layer "B.Cu") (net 4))
 (segment (start 91 73.805578) (end 90.299 73.104578) (width 0.6) (layer "B.Cu") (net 4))
 (segment (start 56.49 40.37) (end 56.5 40.36) (width 0.6) (layer "B.Cu") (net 4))
 (segment (start 89.604578 78.201) (end 91 76.805578) (width 0.6) (layer "B.Cu") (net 4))
 (segment (start 89.915628 81) (end 76.5 81) (width 0.6) (layer "B.Cu") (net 4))
 (segment (start 29.81 58.11) (end 31.7111 58.11) (width 0.6) (layer "B.Cu") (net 4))
 (segment (start 22.19 64) (end 22.19 75.89) (width 0.6) (layer "B.Cu") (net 1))
 (segment (start 21.89 64.3) (end 22.19 64) (width 0.6) (layer "B.Cu") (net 1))
 (segment (start 17 64.3) (end 21.89 64.3) (width 0.6) (layer "B.Cu") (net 1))
 (segment (start 22.19 60.65) (end 22.19 64) (width 0.6) (layer "B.Cu") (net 1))
 (segment (start 16.6975 42.4467) (end 16.6975 26.9025) (width 0.6) (layer "B.Cu") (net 3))
 (segment (start 19.2025 43) (end 17.2508 43) (width 0.6) (layer "B.Cu") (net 3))
 (segment (start 17.2508 43) (end 16.6975 42.4467) (width 0.6) (layer "B.Cu") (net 3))
 (segment (start 16.6975 26.9025) (end 17.1 26.5) (width 0.6) (layer "B.Cu") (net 3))
 (segment (start 17.1 26.5) (end 18.55 26.5) (width 0.6) (layer "B.Cu") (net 3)))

